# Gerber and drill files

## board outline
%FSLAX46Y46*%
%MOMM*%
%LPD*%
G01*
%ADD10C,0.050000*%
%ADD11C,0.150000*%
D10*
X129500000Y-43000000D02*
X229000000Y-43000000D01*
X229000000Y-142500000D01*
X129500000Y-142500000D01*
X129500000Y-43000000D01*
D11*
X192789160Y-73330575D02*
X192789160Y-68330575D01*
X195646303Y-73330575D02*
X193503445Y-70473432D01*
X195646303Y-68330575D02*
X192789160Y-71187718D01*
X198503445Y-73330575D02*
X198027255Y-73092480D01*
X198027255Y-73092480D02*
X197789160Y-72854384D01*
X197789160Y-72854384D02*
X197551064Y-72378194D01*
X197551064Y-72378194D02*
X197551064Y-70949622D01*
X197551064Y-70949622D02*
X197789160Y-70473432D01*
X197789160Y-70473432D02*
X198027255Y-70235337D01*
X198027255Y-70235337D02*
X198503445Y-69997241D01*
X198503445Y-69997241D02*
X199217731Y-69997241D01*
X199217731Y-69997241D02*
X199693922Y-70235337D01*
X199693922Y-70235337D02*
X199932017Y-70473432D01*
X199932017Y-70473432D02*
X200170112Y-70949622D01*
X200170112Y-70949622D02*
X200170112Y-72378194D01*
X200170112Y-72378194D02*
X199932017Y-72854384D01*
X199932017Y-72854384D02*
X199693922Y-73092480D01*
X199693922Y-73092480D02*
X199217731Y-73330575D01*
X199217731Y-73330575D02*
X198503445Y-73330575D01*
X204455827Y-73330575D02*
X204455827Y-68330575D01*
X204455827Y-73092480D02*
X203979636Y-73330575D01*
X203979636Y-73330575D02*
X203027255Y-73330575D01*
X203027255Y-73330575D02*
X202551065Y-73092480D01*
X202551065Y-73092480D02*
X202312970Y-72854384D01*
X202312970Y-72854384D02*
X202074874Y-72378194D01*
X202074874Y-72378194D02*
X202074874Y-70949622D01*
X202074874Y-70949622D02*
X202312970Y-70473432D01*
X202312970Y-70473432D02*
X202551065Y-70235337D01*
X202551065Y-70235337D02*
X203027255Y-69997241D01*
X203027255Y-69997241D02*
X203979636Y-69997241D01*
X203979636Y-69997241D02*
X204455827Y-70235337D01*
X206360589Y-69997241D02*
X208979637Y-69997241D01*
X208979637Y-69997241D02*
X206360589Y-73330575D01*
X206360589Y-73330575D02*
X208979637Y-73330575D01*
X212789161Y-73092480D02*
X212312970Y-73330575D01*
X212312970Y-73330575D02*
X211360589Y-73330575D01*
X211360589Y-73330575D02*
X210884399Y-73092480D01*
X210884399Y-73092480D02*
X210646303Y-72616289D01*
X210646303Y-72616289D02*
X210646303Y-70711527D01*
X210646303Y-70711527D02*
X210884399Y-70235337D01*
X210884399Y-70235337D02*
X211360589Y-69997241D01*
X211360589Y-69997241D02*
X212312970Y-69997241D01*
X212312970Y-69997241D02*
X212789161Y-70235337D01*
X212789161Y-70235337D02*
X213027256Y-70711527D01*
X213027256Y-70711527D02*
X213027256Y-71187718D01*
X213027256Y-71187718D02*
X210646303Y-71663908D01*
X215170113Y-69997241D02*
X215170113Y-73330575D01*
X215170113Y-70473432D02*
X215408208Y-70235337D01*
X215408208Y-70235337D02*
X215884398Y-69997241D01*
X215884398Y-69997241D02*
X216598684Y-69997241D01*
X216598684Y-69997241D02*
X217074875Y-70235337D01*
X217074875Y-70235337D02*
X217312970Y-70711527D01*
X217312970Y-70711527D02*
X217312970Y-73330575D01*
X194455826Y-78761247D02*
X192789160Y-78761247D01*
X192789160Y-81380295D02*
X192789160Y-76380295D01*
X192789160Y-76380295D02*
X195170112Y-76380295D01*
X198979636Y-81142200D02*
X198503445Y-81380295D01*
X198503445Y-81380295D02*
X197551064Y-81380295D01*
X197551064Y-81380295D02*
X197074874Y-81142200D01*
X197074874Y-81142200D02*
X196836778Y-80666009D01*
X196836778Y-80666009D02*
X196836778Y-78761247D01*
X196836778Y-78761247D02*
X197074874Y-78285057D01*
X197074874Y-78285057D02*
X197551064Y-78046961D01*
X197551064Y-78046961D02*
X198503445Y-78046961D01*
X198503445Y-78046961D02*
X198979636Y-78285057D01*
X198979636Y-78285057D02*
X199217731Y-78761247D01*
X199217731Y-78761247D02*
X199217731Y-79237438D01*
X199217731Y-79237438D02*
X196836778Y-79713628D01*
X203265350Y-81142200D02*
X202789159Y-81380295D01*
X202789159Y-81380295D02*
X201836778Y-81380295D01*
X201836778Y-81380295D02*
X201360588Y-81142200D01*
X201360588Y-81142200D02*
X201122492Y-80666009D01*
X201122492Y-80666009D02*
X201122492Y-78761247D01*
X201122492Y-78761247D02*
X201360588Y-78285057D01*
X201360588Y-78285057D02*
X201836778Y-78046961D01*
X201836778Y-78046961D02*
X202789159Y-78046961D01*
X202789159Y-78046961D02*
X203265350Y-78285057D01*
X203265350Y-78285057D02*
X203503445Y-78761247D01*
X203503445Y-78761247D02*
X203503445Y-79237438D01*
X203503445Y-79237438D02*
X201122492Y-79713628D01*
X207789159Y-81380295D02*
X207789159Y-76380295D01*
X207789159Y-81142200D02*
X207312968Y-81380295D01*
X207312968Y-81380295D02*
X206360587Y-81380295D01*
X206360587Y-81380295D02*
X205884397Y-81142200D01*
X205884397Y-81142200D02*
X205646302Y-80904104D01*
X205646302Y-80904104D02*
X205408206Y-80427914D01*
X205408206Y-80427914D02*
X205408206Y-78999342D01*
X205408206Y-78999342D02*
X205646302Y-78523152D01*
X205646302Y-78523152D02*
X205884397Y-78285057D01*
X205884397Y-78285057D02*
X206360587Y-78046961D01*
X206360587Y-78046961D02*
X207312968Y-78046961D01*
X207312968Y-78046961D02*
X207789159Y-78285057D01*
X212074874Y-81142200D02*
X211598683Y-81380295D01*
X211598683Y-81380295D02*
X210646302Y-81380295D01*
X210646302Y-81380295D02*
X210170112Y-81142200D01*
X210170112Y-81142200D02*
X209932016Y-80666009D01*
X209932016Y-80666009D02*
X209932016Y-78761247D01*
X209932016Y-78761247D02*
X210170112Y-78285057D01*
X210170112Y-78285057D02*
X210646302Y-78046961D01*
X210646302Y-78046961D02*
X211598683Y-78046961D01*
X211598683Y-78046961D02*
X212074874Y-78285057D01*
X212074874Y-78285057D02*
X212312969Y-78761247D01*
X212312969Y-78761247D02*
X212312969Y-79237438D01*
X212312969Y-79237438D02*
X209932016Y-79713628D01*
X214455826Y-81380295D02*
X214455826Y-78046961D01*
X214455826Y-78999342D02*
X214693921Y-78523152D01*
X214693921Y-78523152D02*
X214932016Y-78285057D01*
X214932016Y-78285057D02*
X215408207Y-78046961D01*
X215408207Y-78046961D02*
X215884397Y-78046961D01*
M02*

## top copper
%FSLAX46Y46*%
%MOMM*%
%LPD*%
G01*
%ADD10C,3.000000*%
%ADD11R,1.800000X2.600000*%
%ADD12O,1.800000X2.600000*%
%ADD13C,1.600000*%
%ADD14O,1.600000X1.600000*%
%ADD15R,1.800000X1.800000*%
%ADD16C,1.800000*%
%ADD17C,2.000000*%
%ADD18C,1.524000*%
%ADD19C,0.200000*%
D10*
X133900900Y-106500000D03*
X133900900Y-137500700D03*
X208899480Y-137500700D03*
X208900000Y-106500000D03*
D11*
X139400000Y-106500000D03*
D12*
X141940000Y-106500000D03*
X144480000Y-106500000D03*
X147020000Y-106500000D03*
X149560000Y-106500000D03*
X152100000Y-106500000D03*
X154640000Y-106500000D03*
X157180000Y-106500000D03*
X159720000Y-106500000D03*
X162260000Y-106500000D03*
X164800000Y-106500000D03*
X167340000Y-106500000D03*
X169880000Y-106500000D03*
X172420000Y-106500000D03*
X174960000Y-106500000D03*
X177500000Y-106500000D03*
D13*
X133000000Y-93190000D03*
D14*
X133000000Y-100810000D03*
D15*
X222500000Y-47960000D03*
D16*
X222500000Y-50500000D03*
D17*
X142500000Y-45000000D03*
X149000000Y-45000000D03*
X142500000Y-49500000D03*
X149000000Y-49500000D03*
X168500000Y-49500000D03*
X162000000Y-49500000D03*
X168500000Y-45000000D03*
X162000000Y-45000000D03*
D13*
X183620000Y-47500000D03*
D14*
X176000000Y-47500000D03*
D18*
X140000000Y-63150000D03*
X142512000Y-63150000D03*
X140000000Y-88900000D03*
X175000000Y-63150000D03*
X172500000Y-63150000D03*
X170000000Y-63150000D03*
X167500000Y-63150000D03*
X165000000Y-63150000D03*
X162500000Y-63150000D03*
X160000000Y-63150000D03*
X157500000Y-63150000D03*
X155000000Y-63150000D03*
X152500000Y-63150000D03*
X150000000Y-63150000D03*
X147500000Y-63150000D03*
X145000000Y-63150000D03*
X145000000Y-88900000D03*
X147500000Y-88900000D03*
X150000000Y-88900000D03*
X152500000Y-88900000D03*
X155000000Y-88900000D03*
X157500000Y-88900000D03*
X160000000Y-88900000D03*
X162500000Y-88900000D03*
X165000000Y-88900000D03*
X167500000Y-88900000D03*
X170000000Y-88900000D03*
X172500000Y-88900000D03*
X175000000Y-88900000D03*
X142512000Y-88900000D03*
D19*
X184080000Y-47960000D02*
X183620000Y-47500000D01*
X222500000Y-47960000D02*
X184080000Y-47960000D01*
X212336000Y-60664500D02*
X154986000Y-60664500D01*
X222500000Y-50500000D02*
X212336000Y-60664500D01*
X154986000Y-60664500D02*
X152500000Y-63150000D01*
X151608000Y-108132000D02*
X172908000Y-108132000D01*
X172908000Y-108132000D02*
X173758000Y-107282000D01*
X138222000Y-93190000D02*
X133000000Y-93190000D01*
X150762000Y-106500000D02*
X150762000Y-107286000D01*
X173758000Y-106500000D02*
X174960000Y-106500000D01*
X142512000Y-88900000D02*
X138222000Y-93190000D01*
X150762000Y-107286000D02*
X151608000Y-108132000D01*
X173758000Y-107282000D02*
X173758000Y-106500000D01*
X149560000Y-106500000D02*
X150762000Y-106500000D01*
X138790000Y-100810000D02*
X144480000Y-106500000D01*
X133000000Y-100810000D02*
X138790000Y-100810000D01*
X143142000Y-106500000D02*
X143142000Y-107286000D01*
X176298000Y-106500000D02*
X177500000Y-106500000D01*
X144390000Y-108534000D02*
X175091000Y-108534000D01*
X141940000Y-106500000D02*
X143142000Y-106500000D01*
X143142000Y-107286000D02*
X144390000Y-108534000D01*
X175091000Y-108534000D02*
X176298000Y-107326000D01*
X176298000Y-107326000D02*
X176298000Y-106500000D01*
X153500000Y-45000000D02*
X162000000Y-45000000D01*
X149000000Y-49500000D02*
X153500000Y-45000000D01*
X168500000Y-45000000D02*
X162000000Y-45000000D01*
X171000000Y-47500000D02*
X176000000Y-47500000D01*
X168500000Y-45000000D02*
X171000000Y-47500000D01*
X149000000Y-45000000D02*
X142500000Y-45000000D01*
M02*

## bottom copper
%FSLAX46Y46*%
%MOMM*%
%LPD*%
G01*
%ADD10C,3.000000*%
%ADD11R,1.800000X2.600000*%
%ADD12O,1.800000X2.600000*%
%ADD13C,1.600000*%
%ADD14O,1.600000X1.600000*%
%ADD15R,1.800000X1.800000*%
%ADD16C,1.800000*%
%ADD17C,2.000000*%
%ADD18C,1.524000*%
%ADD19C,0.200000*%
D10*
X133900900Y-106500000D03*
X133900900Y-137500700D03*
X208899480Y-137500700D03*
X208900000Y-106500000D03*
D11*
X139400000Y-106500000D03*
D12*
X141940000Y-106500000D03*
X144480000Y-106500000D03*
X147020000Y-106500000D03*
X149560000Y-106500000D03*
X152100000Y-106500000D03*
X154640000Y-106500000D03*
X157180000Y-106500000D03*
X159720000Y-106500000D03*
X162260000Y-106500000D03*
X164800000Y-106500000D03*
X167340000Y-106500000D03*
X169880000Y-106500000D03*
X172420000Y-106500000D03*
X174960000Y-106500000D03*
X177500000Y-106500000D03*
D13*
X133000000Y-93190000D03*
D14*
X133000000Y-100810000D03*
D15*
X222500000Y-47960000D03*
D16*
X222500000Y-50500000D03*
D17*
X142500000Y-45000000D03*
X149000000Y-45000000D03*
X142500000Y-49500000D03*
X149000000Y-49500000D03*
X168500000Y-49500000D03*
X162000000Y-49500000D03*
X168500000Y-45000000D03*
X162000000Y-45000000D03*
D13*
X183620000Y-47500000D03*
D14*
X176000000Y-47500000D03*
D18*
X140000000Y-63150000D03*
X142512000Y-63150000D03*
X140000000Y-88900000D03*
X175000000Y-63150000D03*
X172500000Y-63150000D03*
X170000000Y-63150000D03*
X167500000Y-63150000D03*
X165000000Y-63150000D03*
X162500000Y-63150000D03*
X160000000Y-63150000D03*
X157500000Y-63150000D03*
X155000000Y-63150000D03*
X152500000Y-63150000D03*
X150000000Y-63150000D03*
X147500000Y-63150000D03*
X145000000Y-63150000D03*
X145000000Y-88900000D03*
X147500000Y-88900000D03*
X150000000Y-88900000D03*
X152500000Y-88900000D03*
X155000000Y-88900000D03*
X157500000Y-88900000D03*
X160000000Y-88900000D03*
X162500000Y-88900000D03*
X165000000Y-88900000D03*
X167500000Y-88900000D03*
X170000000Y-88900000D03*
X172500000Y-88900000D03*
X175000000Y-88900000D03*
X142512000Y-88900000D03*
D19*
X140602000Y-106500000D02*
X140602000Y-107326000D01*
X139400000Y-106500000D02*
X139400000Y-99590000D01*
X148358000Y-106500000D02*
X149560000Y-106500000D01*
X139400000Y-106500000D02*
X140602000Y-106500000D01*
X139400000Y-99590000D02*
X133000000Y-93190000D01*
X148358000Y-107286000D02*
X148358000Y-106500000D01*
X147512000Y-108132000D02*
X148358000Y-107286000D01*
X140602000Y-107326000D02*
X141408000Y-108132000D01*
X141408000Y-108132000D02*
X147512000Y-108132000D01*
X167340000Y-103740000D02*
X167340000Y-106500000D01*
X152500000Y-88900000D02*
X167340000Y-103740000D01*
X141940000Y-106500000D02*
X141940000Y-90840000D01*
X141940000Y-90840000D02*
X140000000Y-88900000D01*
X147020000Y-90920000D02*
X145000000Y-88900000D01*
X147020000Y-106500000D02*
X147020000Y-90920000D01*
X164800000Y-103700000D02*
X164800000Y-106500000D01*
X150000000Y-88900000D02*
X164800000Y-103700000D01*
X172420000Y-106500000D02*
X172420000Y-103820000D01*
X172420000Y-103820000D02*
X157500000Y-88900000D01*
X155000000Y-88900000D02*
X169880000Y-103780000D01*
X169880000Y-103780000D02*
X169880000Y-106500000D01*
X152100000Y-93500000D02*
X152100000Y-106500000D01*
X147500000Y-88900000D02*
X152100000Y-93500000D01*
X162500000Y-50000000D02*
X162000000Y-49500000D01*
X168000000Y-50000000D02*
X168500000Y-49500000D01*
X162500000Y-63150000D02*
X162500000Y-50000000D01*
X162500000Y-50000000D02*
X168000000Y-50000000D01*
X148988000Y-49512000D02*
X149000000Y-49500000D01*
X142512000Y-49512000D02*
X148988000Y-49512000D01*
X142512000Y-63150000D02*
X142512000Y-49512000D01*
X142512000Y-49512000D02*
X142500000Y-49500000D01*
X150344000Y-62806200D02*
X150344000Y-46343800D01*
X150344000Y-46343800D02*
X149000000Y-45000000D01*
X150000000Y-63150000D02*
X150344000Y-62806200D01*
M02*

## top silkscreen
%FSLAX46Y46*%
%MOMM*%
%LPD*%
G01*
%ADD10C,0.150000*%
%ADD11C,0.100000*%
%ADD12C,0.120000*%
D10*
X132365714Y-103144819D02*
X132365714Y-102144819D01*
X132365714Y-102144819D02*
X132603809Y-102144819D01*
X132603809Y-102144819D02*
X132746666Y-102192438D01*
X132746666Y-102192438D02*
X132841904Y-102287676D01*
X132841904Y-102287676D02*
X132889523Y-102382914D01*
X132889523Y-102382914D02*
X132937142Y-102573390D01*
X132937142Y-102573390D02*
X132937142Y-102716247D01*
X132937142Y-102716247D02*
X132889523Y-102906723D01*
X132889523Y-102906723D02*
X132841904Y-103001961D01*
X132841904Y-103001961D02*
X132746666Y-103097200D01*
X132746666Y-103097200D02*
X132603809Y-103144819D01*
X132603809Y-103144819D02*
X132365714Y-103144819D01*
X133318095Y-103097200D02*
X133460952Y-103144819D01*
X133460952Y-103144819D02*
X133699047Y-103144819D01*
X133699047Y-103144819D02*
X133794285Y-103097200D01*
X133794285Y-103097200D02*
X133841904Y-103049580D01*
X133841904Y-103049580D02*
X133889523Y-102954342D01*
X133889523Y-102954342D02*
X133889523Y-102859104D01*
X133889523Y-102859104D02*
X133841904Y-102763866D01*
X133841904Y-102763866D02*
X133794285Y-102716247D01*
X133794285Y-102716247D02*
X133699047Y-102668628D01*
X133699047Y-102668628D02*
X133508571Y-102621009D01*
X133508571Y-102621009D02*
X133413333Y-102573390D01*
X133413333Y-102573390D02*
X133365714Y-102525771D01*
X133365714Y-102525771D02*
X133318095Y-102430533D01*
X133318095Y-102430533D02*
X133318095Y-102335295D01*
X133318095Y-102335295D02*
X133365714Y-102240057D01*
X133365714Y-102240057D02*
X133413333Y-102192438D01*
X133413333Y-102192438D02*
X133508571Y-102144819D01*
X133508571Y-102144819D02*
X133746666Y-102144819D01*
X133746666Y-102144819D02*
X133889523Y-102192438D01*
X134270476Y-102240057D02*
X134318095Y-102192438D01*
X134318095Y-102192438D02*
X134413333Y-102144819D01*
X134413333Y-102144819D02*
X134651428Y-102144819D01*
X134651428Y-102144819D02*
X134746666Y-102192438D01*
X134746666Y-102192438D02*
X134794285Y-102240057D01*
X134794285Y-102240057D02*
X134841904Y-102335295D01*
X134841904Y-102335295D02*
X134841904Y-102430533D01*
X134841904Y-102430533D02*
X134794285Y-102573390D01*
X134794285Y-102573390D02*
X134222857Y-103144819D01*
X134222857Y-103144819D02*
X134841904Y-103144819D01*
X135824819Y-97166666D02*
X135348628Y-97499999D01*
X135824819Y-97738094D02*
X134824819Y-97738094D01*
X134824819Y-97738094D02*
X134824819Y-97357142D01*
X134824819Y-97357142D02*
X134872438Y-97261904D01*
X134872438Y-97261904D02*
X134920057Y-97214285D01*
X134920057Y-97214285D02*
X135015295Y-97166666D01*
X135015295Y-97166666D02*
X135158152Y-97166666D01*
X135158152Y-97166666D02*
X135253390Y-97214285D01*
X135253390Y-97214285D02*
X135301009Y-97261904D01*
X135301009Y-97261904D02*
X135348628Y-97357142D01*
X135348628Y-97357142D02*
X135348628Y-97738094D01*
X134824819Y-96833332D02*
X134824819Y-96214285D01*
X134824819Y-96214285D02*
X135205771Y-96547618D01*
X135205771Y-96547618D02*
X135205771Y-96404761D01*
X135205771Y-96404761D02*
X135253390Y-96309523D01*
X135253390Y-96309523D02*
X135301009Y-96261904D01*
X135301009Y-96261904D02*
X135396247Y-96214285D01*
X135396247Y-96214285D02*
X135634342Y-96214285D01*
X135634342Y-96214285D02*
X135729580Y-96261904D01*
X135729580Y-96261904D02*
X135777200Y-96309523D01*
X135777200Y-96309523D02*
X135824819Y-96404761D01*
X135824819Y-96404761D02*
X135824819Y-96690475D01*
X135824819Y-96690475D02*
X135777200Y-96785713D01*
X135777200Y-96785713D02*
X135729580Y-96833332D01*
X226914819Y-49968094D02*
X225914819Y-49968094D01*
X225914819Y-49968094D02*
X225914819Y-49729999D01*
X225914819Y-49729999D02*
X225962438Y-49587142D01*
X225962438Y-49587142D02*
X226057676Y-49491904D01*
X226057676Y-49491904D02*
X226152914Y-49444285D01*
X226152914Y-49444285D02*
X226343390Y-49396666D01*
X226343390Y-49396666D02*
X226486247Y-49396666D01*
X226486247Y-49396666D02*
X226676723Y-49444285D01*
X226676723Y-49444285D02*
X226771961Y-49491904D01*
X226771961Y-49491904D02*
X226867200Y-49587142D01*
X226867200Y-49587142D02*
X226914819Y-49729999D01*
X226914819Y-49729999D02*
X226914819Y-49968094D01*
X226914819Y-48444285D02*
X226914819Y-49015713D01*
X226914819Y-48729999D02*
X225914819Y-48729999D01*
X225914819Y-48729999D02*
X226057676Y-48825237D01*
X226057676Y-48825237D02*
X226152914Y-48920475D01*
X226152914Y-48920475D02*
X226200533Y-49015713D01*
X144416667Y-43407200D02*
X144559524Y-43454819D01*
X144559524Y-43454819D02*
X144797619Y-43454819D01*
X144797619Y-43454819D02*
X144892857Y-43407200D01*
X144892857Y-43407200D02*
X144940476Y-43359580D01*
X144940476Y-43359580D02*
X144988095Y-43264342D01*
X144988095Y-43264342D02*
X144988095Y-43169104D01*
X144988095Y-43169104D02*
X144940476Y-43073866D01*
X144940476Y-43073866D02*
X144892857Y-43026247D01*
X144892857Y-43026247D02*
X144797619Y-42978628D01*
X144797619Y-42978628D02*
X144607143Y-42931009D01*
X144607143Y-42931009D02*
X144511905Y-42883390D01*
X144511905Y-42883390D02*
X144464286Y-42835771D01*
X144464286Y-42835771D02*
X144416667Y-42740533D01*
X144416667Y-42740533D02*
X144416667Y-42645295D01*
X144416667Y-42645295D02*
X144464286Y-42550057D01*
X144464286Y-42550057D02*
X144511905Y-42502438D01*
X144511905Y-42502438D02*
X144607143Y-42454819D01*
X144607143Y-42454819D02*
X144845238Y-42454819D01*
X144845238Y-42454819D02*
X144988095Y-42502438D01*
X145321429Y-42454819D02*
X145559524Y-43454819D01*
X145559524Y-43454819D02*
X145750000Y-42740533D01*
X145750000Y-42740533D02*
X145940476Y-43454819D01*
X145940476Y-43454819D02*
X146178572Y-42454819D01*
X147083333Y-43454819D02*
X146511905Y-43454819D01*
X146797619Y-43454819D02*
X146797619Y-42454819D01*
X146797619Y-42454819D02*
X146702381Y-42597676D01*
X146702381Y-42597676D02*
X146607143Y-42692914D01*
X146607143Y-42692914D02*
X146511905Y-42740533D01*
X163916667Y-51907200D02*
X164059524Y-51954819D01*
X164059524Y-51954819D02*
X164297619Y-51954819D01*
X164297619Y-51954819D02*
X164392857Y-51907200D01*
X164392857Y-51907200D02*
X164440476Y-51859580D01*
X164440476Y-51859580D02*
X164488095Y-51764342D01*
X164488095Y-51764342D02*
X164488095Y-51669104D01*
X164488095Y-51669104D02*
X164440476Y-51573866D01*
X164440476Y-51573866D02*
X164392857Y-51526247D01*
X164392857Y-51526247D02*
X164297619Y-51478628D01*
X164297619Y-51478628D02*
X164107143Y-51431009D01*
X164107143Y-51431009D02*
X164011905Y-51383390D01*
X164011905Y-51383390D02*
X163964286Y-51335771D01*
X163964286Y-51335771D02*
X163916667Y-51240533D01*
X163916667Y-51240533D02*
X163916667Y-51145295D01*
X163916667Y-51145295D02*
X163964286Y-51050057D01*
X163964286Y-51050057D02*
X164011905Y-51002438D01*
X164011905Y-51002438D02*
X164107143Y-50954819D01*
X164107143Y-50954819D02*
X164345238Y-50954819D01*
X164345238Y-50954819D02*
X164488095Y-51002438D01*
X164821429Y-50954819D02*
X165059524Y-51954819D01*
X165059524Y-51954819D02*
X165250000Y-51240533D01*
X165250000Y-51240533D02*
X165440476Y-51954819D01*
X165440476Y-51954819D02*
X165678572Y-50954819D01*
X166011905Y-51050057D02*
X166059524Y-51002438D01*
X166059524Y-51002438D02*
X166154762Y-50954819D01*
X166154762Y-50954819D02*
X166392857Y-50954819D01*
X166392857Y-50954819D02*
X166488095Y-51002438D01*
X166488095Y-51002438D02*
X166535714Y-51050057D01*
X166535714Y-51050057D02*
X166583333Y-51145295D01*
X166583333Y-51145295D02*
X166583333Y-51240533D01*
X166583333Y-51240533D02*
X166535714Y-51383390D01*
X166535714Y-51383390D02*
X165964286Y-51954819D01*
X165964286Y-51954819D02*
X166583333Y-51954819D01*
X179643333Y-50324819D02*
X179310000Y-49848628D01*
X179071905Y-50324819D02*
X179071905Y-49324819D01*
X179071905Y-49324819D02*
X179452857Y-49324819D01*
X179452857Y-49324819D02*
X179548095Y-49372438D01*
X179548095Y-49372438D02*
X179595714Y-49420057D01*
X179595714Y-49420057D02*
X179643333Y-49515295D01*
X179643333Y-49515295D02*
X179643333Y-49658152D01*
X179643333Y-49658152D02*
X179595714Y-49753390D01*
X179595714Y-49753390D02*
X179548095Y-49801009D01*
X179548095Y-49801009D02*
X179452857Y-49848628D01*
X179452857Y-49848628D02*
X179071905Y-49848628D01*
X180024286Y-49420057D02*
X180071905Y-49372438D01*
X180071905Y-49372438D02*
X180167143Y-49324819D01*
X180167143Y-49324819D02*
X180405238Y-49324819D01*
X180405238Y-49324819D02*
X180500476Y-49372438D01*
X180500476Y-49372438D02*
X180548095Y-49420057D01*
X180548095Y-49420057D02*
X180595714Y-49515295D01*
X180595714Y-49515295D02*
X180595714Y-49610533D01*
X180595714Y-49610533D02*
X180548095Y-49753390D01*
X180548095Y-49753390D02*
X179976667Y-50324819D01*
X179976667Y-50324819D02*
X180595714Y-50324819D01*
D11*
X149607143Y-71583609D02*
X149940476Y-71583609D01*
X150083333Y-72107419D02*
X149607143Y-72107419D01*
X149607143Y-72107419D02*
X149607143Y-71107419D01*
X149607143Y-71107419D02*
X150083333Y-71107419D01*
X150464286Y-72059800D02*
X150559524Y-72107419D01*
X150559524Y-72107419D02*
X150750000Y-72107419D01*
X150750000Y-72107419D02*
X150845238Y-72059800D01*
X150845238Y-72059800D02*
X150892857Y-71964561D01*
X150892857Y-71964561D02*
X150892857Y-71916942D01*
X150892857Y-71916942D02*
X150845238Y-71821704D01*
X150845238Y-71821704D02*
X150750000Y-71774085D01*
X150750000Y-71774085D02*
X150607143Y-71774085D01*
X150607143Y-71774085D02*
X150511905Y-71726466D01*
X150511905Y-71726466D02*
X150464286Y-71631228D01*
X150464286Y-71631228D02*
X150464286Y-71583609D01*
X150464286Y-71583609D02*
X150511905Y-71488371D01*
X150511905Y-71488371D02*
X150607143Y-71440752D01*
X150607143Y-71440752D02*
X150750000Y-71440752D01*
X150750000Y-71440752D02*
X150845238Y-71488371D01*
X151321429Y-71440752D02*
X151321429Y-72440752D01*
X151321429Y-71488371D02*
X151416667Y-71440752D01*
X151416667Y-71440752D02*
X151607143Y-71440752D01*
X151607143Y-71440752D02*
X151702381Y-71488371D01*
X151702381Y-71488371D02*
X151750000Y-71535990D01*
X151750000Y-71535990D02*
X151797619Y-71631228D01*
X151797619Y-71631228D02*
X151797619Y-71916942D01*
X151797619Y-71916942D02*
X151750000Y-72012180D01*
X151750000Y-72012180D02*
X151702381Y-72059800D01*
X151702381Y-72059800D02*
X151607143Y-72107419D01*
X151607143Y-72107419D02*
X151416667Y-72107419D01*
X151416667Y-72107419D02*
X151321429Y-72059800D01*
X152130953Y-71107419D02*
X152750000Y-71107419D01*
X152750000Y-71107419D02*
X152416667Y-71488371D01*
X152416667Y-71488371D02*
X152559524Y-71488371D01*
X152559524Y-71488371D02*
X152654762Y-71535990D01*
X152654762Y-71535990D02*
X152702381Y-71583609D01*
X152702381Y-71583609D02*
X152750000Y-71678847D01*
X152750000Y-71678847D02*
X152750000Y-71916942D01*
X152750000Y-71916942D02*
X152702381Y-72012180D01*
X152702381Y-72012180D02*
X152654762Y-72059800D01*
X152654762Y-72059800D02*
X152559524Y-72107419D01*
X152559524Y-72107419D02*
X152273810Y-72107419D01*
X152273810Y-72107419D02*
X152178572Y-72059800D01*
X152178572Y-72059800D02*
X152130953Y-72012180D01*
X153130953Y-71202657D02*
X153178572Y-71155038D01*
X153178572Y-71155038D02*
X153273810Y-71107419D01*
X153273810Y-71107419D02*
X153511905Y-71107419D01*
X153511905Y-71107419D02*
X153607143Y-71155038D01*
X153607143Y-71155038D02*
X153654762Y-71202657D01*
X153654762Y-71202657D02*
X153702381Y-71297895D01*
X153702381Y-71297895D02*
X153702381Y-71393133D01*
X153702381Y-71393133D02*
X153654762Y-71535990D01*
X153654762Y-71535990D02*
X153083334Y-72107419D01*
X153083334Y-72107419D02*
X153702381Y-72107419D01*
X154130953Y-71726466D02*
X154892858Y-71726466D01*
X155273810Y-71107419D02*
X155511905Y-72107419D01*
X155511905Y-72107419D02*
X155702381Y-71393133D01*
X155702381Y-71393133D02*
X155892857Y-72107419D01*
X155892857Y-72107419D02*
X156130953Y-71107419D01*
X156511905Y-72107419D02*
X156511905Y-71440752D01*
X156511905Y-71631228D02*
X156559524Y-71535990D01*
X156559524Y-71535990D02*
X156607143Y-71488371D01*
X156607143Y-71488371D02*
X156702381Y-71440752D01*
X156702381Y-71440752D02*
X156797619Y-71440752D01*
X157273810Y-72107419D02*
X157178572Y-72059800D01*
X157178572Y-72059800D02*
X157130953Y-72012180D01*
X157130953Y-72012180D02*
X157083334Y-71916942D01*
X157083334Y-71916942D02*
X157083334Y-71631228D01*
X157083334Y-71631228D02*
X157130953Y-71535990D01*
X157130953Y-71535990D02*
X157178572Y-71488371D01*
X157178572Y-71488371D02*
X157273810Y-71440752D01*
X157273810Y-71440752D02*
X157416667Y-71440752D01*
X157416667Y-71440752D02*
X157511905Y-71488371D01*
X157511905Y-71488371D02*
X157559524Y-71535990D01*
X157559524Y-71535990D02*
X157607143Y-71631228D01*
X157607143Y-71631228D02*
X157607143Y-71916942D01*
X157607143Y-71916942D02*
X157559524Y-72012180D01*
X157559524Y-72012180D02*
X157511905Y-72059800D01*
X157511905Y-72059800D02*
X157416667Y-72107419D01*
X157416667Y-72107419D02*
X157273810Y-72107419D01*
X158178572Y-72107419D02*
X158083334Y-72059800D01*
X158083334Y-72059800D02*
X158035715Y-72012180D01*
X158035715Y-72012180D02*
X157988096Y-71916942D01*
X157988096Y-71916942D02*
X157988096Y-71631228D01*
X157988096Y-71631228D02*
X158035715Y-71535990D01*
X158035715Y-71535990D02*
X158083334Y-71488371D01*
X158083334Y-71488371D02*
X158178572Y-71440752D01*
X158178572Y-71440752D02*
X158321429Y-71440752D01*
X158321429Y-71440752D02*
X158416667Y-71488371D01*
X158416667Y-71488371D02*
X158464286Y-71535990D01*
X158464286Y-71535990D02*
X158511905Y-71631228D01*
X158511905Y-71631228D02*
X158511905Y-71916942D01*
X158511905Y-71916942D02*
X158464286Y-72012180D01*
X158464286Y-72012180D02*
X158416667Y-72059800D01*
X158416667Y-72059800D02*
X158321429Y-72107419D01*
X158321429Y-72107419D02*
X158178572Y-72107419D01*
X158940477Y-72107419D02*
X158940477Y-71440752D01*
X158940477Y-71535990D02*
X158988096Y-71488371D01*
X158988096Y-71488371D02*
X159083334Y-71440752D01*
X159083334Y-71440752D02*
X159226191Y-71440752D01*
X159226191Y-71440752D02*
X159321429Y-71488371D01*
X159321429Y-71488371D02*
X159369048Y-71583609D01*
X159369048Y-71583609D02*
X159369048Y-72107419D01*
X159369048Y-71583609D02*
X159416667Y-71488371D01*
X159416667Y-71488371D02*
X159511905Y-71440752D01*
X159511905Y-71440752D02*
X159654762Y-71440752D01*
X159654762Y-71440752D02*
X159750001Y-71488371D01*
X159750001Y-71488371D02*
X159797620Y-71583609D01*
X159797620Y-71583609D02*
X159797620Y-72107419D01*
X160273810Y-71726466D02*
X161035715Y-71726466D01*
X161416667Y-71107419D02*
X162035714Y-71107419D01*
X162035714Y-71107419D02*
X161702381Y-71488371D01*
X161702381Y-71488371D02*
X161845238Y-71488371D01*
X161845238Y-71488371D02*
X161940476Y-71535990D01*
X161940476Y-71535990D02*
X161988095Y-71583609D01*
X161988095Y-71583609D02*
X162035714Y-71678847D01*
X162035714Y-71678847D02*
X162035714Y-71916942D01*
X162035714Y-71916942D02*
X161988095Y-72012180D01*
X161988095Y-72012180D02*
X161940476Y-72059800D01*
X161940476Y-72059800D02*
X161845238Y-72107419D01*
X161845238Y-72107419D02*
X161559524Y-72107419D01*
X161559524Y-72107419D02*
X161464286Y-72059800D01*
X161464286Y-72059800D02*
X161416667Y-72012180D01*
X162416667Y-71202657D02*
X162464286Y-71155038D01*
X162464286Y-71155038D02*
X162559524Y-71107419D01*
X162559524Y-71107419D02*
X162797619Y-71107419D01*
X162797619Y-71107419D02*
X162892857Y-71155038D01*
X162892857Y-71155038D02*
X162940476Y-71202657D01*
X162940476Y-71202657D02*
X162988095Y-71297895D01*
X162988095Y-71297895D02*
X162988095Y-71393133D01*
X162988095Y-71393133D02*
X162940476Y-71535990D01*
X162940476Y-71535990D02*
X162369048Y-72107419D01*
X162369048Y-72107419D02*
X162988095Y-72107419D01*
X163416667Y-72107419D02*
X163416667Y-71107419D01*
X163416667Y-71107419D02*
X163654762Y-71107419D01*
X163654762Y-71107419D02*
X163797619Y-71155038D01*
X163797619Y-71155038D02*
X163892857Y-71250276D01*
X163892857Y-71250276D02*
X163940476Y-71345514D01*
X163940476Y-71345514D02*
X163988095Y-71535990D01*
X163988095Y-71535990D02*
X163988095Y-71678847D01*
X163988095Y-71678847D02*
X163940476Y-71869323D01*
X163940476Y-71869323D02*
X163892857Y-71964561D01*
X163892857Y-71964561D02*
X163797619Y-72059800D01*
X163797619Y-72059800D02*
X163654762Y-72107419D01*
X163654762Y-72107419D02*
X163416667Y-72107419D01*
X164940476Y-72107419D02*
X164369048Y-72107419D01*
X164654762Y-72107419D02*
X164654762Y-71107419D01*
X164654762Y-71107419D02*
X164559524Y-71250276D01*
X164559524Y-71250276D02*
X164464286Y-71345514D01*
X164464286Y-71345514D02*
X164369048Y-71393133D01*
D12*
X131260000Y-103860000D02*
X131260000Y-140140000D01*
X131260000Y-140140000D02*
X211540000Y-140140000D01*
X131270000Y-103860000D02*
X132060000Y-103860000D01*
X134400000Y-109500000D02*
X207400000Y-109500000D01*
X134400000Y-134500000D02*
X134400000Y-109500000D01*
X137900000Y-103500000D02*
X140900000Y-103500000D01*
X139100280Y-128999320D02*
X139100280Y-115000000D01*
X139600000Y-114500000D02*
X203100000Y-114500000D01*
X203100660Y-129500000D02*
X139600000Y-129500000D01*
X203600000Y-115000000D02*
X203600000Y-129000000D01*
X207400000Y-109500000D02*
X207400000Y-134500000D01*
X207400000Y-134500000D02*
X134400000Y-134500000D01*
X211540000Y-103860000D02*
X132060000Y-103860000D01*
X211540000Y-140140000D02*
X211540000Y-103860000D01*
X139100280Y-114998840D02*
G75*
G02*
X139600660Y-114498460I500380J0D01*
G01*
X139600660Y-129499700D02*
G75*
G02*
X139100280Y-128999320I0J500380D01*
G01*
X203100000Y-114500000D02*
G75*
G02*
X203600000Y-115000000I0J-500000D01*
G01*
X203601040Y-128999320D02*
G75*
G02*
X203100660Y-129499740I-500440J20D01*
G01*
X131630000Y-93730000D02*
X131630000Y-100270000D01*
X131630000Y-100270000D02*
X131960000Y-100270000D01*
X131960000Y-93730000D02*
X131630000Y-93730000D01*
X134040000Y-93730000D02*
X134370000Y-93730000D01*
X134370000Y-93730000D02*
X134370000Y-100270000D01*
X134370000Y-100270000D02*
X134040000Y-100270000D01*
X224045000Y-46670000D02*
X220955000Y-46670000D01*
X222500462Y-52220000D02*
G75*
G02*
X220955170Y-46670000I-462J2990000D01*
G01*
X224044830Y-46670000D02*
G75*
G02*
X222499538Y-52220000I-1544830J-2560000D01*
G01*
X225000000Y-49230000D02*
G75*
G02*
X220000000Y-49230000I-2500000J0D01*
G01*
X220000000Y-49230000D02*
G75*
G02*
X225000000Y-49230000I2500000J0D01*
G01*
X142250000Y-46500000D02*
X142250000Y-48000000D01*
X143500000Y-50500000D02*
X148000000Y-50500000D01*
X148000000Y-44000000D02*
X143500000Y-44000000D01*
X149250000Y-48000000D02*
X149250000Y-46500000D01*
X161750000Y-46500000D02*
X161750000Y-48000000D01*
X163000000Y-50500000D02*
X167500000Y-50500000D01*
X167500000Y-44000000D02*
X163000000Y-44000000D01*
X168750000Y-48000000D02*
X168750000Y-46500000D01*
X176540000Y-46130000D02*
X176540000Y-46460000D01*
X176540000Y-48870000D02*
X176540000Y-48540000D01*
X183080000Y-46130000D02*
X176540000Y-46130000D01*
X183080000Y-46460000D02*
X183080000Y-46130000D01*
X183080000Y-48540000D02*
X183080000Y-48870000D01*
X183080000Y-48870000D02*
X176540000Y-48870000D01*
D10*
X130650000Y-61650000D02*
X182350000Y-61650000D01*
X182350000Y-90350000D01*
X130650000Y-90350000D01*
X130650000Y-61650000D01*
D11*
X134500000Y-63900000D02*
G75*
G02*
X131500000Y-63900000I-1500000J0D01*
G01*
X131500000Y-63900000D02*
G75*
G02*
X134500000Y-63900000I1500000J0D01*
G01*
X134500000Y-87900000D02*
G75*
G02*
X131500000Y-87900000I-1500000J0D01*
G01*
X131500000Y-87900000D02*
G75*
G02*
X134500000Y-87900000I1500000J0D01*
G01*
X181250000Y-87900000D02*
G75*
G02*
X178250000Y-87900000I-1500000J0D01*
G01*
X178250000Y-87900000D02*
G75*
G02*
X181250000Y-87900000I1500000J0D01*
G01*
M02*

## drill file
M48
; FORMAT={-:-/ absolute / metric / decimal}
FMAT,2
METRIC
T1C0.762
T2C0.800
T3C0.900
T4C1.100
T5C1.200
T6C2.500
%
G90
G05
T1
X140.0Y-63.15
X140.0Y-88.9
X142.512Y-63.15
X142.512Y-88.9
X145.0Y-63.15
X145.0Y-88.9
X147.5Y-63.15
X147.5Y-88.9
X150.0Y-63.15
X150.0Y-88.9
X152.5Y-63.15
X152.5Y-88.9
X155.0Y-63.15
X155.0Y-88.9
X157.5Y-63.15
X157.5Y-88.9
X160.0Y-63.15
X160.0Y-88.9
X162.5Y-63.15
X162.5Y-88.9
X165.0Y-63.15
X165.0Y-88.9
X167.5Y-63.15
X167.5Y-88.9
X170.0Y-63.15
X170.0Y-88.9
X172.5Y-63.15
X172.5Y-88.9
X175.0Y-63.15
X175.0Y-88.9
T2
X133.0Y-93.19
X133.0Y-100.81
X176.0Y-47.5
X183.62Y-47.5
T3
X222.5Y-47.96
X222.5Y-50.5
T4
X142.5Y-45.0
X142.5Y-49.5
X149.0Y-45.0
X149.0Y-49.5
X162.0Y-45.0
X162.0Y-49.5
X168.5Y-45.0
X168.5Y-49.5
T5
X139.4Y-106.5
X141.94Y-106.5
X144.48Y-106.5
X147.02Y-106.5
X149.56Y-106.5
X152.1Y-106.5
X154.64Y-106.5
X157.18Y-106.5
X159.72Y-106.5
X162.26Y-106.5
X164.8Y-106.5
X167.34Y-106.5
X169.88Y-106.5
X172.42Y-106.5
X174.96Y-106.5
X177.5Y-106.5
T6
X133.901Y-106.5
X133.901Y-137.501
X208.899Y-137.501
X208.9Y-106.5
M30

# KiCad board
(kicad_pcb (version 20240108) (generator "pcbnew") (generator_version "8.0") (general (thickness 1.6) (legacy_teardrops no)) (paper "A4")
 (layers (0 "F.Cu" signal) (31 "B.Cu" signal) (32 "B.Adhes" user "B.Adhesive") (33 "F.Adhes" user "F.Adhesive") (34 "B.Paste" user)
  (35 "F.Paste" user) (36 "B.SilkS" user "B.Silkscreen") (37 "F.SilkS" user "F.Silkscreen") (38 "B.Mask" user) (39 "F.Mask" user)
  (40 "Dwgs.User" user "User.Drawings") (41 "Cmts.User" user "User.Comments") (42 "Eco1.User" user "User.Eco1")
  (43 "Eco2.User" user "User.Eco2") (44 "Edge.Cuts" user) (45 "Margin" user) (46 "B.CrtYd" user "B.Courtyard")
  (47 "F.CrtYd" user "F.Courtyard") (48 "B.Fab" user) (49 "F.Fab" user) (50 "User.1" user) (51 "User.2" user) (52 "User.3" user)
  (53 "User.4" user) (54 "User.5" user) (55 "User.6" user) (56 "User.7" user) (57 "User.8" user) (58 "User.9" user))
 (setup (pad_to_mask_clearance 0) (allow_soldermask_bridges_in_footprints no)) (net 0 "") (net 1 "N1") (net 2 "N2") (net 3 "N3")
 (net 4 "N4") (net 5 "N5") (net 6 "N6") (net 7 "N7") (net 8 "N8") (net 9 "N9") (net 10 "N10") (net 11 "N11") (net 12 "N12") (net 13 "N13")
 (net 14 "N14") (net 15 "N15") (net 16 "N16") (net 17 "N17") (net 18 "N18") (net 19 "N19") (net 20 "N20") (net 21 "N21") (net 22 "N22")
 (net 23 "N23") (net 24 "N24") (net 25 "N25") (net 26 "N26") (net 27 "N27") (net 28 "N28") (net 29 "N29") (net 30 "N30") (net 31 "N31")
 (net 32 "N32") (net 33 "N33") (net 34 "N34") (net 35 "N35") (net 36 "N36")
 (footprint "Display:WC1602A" (layer "F.Cu") (at 139.4 106.5)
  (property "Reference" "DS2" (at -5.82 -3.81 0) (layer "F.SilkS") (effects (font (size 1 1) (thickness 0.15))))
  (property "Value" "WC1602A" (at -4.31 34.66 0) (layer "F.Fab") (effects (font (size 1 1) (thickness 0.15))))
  (fp_line (start -8.14 -2.64) (end -8.14 33.64) (stroke (width 0.12) (type solid)) (layer "F.SilkS"))
  (fp_line (start -8.14 33.64) (end 72.14 33.64) (stroke (width 0.12) (type solid)) (layer "F.SilkS"))
  (fp_line (start -8.13 -2.64) (end -7.34 -2.64) (stroke (width 0.12) (type solid)) (layer "F.SilkS"))
  (fp_line (start -5 3) (end 68 3) (stroke (width 0.12) (type solid)) (layer "F.SilkS"))
  (fp_line (start -5 28) (end -5 3) (stroke (width 0.12) (type solid)) (layer "F.SilkS"))
  (fp_line (start -1.5 -3) (end 1.5 -3) (stroke (width 0.12) (type solid)) (layer "F.SilkS"))
  (fp_line (start -0.29972 22.49932) (end -0.29972 8.5) (stroke (width 0.12) (type solid)) (layer "F.SilkS"))
  (fp_line (start 0.2 8) (end 63.7 8) (stroke (width 0.12) (type solid)) (layer "F.SilkS"))
  (fp_line (start 63.70066 23) (end 0.2 23) (stroke (width 0.12) (type solid)) (layer "F.SilkS"))
  (fp_line (start 64.2 8.5) (end 64.2 22.5) (stroke (width 0.12) (type solid)) (layer "F.SilkS"))
  (fp_line (start 68 3) (end 68 28) (stroke (width 0.12) (type solid)) (layer "F.SilkS"))
  (fp_line (start 68 28) (end -5 28) (stroke (width 0.12) (type solid)) (layer "F.SilkS"))
  (fp_line (start 72.14 -2.64) (end -7.34 -2.64) (stroke (width 0.12) (type solid)) (layer "F.SilkS"))
  (fp_line (start 72.14 33.64) (end 72.14 -2.64) (stroke (width 0.12) (type solid)) (layer "F.SilkS"))
  (fp_arc (start -0.29972 8.49884) (mid -0.153162 8.145018) (end 0.20066 7.99846) (stroke (width 0.12) (type solid)) (layer "F.SilkS"))
  (fp_arc (start 0.20066 22.9997) (mid -0.153162 22.853142) (end -0.29972 22.49932) (stroke (width 0.12) (type solid)) (layer "F.SilkS"))
  (fp_arc (start 63.7 8) (mid 64.053553 8.146447) (end 64.2 8.5) (stroke (width 0.12) (type solid)) (layer "F.SilkS"))
  (fp_arc (start 64.20104 22.49932) (mid 64.054473 22.853115) (end 63.70066 22.9997) (stroke (width 0.12) (type solid)) (layer "F.SilkS"))
  (pad "" thru_hole circle (at -5.4991 0) (size 3 3) (drill 2.5) (layers "*.Cu" "*.Mask") (remove_unused_layers no))
  (pad "" thru_hole circle (at -5.4991 31.0007) (size 3 3) (drill 2.5) (layers "*.Cu" "*.Mask") (remove_unused_layers no))
  (pad "" thru_hole circle (at 69.49948 31.0007) (size 3 3) (drill 2.5) (layers "*.Cu" "*.Mask") (remove_unused_layers no))
  (pad "" thru_hole circle (at 69.5 0) (size 3 3) (drill 2.5) (layers "*.Cu" "*.Mask") (remove_unused_layers no))
  (pad "1" thru_hole rect (at 0 0) (size 1.8 2.6) (drill 1.2) (layers "*.Cu" "*.Mask") (remove_unused_layers no) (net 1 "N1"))
  (pad "2" thru_hole oval (at 2.54 0) (size 1.8 2.6) (drill 1.2) (layers "*.Cu" "*.Mask") (remove_unused_layers no) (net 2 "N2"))
  (pad "3" thru_hole oval (at 5.08 0) (size 1.8 2.6) (drill 1.2) (layers "*.Cu" "*.Mask") (remove_unused_layers no) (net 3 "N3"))
  (pad "4" thru_hole oval (at 7.62 0) (size 1.8 2.6) (drill 1.2) (layers "*.Cu" "*.Mask") (remove_unused_layers no) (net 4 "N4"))
  (pad "5" thru_hole oval (at 10.16 0) (size 1.8 2.6) (drill 1.2) (layers "*.Cu" "*.Mask") (remove_unused_layers no) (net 1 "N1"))
  (pad "6" thru_hole oval (at 12.7 0) (size 1.8 2.6) (drill 1.2) (layers "*.Cu" "*.Mask") (remove_unused_layers no) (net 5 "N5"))
  (pad "7" thru_hole oval (at 15.24 0) (size 1.8 2.6) (drill 1.2) (layers "*.Cu" "*.Mask") (remove_unused_layers no) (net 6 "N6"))
  (pad "8" thru_hole oval (at 17.78 0) (size 1.8 2.6) (drill 1.2) (layers "*.Cu" "*.Mask") (remove_unused_layers no) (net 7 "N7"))
  (pad "9" thru_hole oval (at 20.32 0) (size 1.8 2.6) (drill 1.2) (layers "*.Cu" "*.Mask") (remove_unused_layers no) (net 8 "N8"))
  (pad "10" thru_hole oval (at 22.86 0) (size 1.8 2.6) (drill 1.2) (layers "*.Cu" "*.Mask") (remove_unused_layers no) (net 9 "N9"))
  (pad "11" thru_hole oval (at 25.4 0) (size 1.8 2.6) (drill 1.2) (layers "*.Cu" "*.Mask") (remove_unused_layers no) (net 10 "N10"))
  (pad "12" thru_hole oval (at 27.94 0) (size 1.8 2.6) (drill 1.2) (layers "*.Cu" "*.Mask") (remove_unused_layers no) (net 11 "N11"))
  (pad "13" thru_hole oval (at 30.48 0) (size 1.8 2.6) (drill 1.2) (layers "*.Cu" "*.Mask") (remove_unused_layers no) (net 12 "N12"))
  (pad "14" thru_hole oval (at 33.02 0) (size 1.8 2.6) (drill 1.2) (layers "*.Cu" "*.Mask") (remove_unused_layers no) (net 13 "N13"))
  (pad "15" thru_hole oval (at 35.56 0) (size 1.8 2.6) (drill 1.2) (layers "*.Cu" "*.Mask") (remove_unused_layers no) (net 1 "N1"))
  (pad "16" thru_hole oval (at 38.1 0) (size 1.8 2.6) (drill 1.2) (layers "*.Cu" "*.Mask") (remove_unused_layers no) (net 2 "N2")))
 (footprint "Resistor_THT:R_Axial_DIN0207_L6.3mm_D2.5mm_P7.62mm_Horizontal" (layer "F.Cu") (at 133 93.19 -90)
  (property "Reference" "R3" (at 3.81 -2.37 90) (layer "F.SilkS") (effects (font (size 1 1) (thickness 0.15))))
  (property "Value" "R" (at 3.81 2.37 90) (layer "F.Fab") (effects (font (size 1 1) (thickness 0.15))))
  (fp_line (start 0.54 1.37) (end 7.08 1.37) (stroke (width 0.12) (type solid)) (layer "F.SilkS"))
  (fp_line (start 7.08 1.37) (end 7.08 1.04) (stroke (width 0.12) (type solid)) (layer "F.SilkS"))
  (fp_line (start 0.54 1.04) (end 0.54 1.37) (stroke (width 0.12) (type solid)) (layer "F.SilkS"))
  (fp_line (start 0.54 -1.04) (end 0.54 -1.37) (stroke (width 0.12) (type solid)) (layer "F.SilkS"))
  (fp_line (start 0.54 -1.37) (end 7.08 -1.37) (stroke (width 0.12) (type solid)) (layer "F.SilkS"))
  (fp_line (start 7.08 -1.37) (end 7.08 -1.04) (stroke (width 0.12) (type solid)) (layer "F.SilkS"))
  (pad "1" thru_hole circle (at 0 0 270) (size 1.6 1.6) (drill 0.8) (layers "*.Cu" "*.Mask") (remove_unused_layers no) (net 1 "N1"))
  (pad "2" thru_hole oval (at 7.62 0 270) (size 1.6 1.6) (drill 0.8) (layers "*.Cu" "*.Mask") (remove_unused_layers no) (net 3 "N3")))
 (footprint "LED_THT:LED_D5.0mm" (layer "F.Cu") (at 222.5 47.96 -90)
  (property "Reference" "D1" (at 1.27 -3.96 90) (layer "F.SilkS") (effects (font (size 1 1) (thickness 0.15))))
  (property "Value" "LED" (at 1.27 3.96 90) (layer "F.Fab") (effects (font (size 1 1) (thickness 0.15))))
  (fp_line (start -1.29 -1.545) (end -1.29 1.545) (stroke (width 0.12) (type solid)) (layer "F.SilkS"))
  (fp_arc (start 4.26 -0.000462) (mid 2.072002 2.880433) (end -1.29 1.54483) (stroke (width 0.12) (type solid)) (layer "F.SilkS"))
  (fp_arc (start -1.29 -1.54483) (mid 2.072002 -2.880433) (end 4.26 0.000462) (stroke (width 0.12) (type solid)) (layer "F.SilkS"))
  (fp_circle (center 1.27 0) (end 3.77 0) (stroke (width 0.12) (type solid)) (fill none) (layer "F.SilkS"))
  (pad "1" thru_hole rect (at 0 0 270) (size 1.8 1.8) (drill 0.9) (layers "*.Cu" "*.Mask") (remove_unused_layers no) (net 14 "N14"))
  (pad "2" thru_hole circle (at 2.54 0 270) (size 1.8 1.8) (drill 0.9) (layers "*.Cu" "*.Mask") (remove_unused_layers no) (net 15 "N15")))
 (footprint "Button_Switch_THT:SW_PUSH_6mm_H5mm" (layer "F.Cu") (at 142.5 45)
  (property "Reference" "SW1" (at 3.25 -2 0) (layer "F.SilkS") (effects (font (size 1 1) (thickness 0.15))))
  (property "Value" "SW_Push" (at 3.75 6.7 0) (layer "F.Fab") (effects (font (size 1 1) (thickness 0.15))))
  (fp_line (start -0.25 1.5) (end -0.25 3) (stroke (width 0.12) (type solid)) (layer "F.SilkS"))
  (fp_line (start 1 5.5) (end 5.5 5.5) (stroke (width 0.12) (type solid)) (layer "F.SilkS"))
  (fp_line (start 5.5 -1) (end 1 -1) (stroke (width 0.12) (type solid)) (layer "F.SilkS"))
  (fp_line (start 6.75 3) (end 6.75 1.5) (stroke (width 0.12) (type solid)) (layer "F.SilkS"))
  (pad "1" thru_hole circle (at 0 0 90) (size 2 2) (drill 1.1) (layers "*.Cu" "*.Mask") (remove_unused_layers no) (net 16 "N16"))
  (pad "1" thru_hole circle (at 6.5 0 90) (size 2 2) (drill 1.1) (layers "*.Cu" "*.Mask") (remove_unused_layers no) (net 16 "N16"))
  (pad "2" thru_hole circle (at 0 4.5 90) (size 2 2) (drill 1.1) (layers "*.Cu" "*.Mask") (remove_unused_layers no) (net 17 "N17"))
  (pad "2" thru_hole circle (at 6.5 4.5 90) (size 2 2) (drill 1.1) (layers "*.Cu" "*.Mask") (remove_unused_layers no) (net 17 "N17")))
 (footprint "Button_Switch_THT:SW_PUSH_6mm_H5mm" (layer "F.Cu") (at 168.5 49.5 180)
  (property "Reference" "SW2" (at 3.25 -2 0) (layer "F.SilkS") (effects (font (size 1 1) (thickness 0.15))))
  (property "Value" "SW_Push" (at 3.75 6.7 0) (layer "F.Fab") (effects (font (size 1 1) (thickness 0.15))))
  (fp_line (start 6.75 3) (end 6.75 1.5) (stroke (width 0.12) (type solid)) (layer "F.SilkS"))
  (fp_line (start 5.5 -1) (end 1 -1) (stroke (width 0.12) (type solid)) (layer "F.SilkS"))
  (fp_line (start 1 5.5) (end 5.5 5.5) (stroke (width 0.12) (type solid)) (layer "F.SilkS"))
  (fp_line (start -0.25 1.5) (end -0.25 3) (stroke (width 0.12) (type solid)) (layer "F.SilkS"))
  (pad "1" thru_hole circle (at 0 0 270) (size 2 2) (drill 1.1) (layers "*.Cu" "*.Mask") (remove_unused_layers no) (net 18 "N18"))
  (pad "1" thru_hole circle (at 6.5 0 270) (size 2 2) (drill 1.1) (layers "*.Cu" "*.Mask") (remove_unused_layers no) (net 18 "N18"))
  (pad "2" thru_hole circle (at 0 4.5 270) (size 2 2) (drill 1.1) (layers "*.Cu" "*.Mask") (remove_unused_layers no) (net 17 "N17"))
  (pad "2" thru_hole circle (at 6.5 4.5 270) (size 2 2) (drill 1.1) (layers "*.Cu" "*.Mask") (remove_unused_layers no) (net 17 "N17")))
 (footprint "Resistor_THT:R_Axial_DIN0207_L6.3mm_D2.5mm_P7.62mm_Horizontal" (layer "F.Cu") (at 183.62 47.5 180)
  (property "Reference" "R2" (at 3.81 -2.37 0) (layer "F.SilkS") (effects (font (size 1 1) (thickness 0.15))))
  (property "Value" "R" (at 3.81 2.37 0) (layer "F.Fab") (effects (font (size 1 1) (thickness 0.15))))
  (fp_line (start 7.08 1.37) (end 7.08 1.04) (stroke (width 0.12) (type solid)) (layer "F.SilkS"))
  (fp_line (start 7.08 -1.37) (end 7.08 -1.04) (stroke (width 0.12) (type solid)) (layer "F.SilkS"))
  (fp_line (start 0.54 1.37) (end 7.08 1.37) (stroke (width 0.12) (type solid)) (layer "F.SilkS"))
  (fp_line (start 0.54 1.04) (end 0.54 1.37) (stroke (width 0.12) (type solid)) (layer "F.SilkS"))
  (fp_line (start 0.54 -1.04) (end 0.54 -1.37) (stroke (width 0.12) (type solid)) (layer "F.SilkS"))
  (fp_line (start 0.54 -1.37) (end 7.08 -1.37) (stroke (width 0.12) (type solid)) (layer "F.SilkS"))
  (pad "1" thru_hole circle (at 0 0 180) (size 1.6 1.6) (drill 0.8) (layers "*.Cu" "*.Mask") (remove_unused_layers no) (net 14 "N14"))
  (pad "2" thru_hole oval (at 7.62 0 180) (size 1.6 1.6) (drill 0.8) (layers "*.Cu" "*.Mask") (remove_unused_layers no) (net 17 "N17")))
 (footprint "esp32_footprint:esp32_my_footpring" (layer "F.Cu") (at 157.25 72.15)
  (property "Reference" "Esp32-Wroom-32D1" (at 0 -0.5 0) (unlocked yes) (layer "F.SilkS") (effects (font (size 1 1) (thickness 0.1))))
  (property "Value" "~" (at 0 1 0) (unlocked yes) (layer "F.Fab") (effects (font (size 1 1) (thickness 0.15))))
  (fp_rect (start -26.6 -10.5) (end 25.1 18.2) (stroke (width 0.15) (type default)) (fill none) (layer "F.SilkS"))
  (fp_circle (center -24.25 -8.25) (end -22.75 -8.25) (stroke (width 0.1) (type default)) (fill none) (layer "F.SilkS"))
  (fp_circle (center -24.25 15.75) (end -22.75 15.75) (stroke (width 0.1) (type default)) (fill none) (layer "F.SilkS"))
  (fp_circle (center 22.5 15.75) (end 24 15.75) (stroke (width 0.1) (type default)) (fill none) (layer "F.SilkS"))
  (pad "0" thru_hole circle (at -17.25 -9) (size 1.524 1.524) (drill 0.762) (layers "*.Cu" "*.Mask") (remove_unused_layers no)
   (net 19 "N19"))
  (pad "1" thru_hole circle (at -14.738 -9) (size 1.524 1.524) (drill 0.762) (layers "*.Cu" "*.Mask") (remove_unused_layers no)
   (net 17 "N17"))
  (pad "2" thru_hole circle (at -17.25 16.75) (size 1.524 1.524) (drill 0.762) (layers "*.Cu" "*.Mask") (remove_unused_layers no)
   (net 2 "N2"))
  (pad "3" thru_hole circle (at 17.75 -9) (size 1.524 1.524) (drill 0.762) (layers "*.Cu" "*.Mask") (remove_unused_layers no) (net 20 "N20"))
  (pad "4" thru_hole circle (at 15.25 -9) (size 1.524 1.524) (drill 0.762) (layers "*.Cu" "*.Mask") (remove_unused_layers no) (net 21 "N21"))
  (pad "5" thru_hole circle (at 12.75 -9) (size 1.524 1.524) (drill 0.762) (layers "*.Cu" "*.Mask") (remove_unused_layers no) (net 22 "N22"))
  (pad "6" thru_hole circle (at 10.25 -9) (size 1.524 1.524) (drill 0.762) (layers "*.Cu" "*.Mask") (remove_unused_layers no) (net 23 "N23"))
  (pad "7" thru_hole circle (at 7.75 -9) (size 1.524 1.524) (drill 0.762) (layers "*.Cu" "*.Mask") (remove_unused_layers no) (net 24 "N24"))
  (pad "8" thru_hole circle (at 5.25 -9) (size 1.524 1.524) (drill 0.762) (layers "*.Cu" "*.Mask") (remove_unused_layers no) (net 18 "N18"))
  (pad "9" thru_hole circle (at 2.75 -9) (size 1.524 1.524) (drill 0.762) (layers "*.Cu" "*.Mask") (remove_unused_layers no) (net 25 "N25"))
  (pad "10" thru_hole circle (at 0.25 -9) (size 1.524 1.524) (drill 0.762) (layers "*.Cu" "*.Mask") (remove_unused_layers no) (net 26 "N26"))
  (pad "11" thru_hole circle (at -2.25 -9) (size 1.524 1.524) (drill 0.762) (layers "*.Cu" "*.Mask") (remove_unused_layers no)
   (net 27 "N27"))
  (pad "12" thru_hole circle (at -4.75 -9) (size 1.524 1.524) (drill 0.762) (layers "*.Cu" "*.Mask") (remove_unused_layers no)
   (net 15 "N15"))
  (pad "13" thru_hole circle (at -7.25 -9) (size 1.524 1.524) (drill 0.762) (layers "*.Cu" "*.Mask") (remove_unused_layers no)
   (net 16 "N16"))
  (pad "14" thru_hole circle (at -9.75 -9) (size 1.524 1.524) (drill 0.762) (layers "*.Cu" "*.Mask") (remove_unused_layers no)
   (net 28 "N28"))
  (pad "16" thru_hole circle (at -12.25 -9) (size 1.524 1.524) (drill 0.762) (layers "*.Cu" "*.Mask") (remove_unused_layers no)
   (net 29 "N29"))
  (pad "23" thru_hole circle (at -12.25 16.75) (size 1.524 1.524) (drill 0.762) (layers "*.Cu" "*.Mask") (remove_unused_layers no)
   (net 4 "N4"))
  (pad "24" thru_hole circle (at -9.75 16.75) (size 1.524 1.524) (drill 0.762) (layers "*.Cu" "*.Mask") (remove_unused_layers no)
   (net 5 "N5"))
  (pad "26" thru_hole circle (at -7.25 16.75) (size 1.524 1.524) (drill 0.762) (layers "*.Cu" "*.Mask") (remove_unused_layers no)
   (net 10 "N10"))
  (pad "27" thru_hole circle (at -4.75 16.75) (size 1.524 1.524) (drill 0.762) (layers "*.Cu" "*.Mask") (remove_unused_layers no)
   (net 11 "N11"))
  (pad "28" thru_hole circle (at -2.25 16.75) (size 1.524 1.524) (drill 0.762) (layers "*.Cu" "*.Mask") (remove_unused_layers no)
   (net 12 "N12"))
  (pad "29" thru_hole circle (at 0.25 16.75) (size 1.524 1.524) (drill 0.762) (layers "*.Cu" "*.Mask") (remove_unused_layers no)
   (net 13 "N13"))
  (pad "30" thru_hole circle (at 2.75 16.75) (size 1.524 1.524) (drill 0.762) (layers "*.Cu" "*.Mask") (remove_unused_layers no)
   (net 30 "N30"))
  (pad "31" thru_hole circle (at 5.25 16.75) (size 1.524 1.524) (drill 0.762) (layers "*.Cu" "*.Mask") (remove_unused_layers no)
   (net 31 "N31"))
  (pad "33" thru_hole circle (at 7.75 16.75) (size 1.524 1.524) (drill 0.762) (layers "*.Cu" "*.Mask") (remove_unused_layers no)
   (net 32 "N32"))
  (pad "34" thru_hole circle (at 10.25 16.75) (size 1.524 1.524) (drill 0.762) (layers "*.Cu" "*.Mask") (remove_unused_layers no)
   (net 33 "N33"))
  (pad "35" thru_hole circle (at 12.75 16.75) (size 1.524 1.524) (drill 0.762) (layers "*.Cu" "*.Mask") (remove_unused_layers no)
   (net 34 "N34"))
  (pad "36" thru_hole circle (at 15.25 16.75) (size 1.524 1.524) (drill 0.762) (layers "*.Cu" "*.Mask") (remove_unused_layers no)
   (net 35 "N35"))
  (pad "37" thru_hole circle (at 17.75 16.75) (size 1.524 1.524) (drill 0.762) (layers "*.Cu" "*.Mask") (remove_unused_layers no)
   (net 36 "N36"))
  (pad "38" thru_hole circle (at -14.738 16.75) (size 1.524 1.524) (drill 0.762) (layers "*.Cu" "*.Mask") (remove_unused_layers no)
   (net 1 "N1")))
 (gr_rect (start 129.5 43) (end 229 142.5) (locked yes) (stroke (width 0.05) (type default)) (fill none) (layer "Edge.Cuts"))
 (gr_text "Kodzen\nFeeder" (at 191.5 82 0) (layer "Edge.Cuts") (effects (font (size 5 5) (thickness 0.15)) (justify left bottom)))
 (segment (start 184.08 47.96) (end 183.62 47.5) (width 0.2) (layer "F.Cu") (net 14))
 (segment (start 222.5 47.96) (end 184.08 47.96) (width 0.2) (layer "F.Cu") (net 14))
 (segment (start 212.336 60.6645) (end 154.986 60.6645) (width 0.2) (layer "F.Cu") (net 15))
 (segment (start 222.5 50.5) (end 212.336 60.6645) (width 0.2) (layer "F.Cu") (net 15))
 (segment (start 154.986 60.6645) (end 152.5 63.15) (width 0.2) (layer "F.Cu") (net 15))
 (segment (start 151.608 108.132) (end 172.908 108.132) (width 0.2) (layer "F.Cu") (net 1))
 (segment (start 172.908 108.132) (end 173.758 107.282) (width 0.2) (layer "F.Cu") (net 1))
 (segment (start 138.222 93.19) (end 133 93.19) (width 0.2) (layer "F.Cu") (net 1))
 (segment (start 150.762 106.5) (end 150.762 107.286) (width 0.2) (layer "F.Cu") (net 1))
 (segment (start 173.758 106.5) (end 174.96 106.5) (width 0.2) (layer "F.Cu") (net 1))
 (segment (start 142.512 88.9) (end 138.222 93.19) (width 0.2) (layer "F.Cu") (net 1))
 (segment (start 150.762 107.286) (end 151.608 108.132) (width 0.2) (layer "F.Cu") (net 1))
 (segment (start 173.758 107.282) (end 173.758 106.5) (width 0.2) (layer "F.Cu") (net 1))
 (segment (start 149.56 106.5) (end 150.762 106.5) (width 0.2) (layer "F.Cu") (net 1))
 (segment (start 140.602 106.5) (end 140.602 107.326) (width 0.2) (layer "B.Cu") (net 1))
 (segment (start 139.4 106.5) (end 139.4 99.59) (width 0.2) (layer "B.Cu") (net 1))
 (segment (start 148.358 106.5) (end 149.56 106.5) (width 0.2) (layer "B.Cu") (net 1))
 (segment (start 139.4 106.5) (end 140.602 106.5) (width 0.2) (layer "B.Cu") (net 1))
 (segment (start 139.4 99.59) (end 133 93.19) (width 0.2) (layer "B.Cu") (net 1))
 (segment (start 148.358 107.286) (end 148.358 106.5) (width 0.2) (layer "B.Cu") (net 1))
 (segment (start 147.512 108.132) (end 148.358 107.286) (width 0.2) (layer "B.Cu") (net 1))
 (segment (start 140.602 107.326) (end 141.408 108.132) (width 0.2) (layer "B.Cu") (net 1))
 (segment (start 141.408 108.132) (end 147.512 108.132) (width 0.2) (layer "B.Cu") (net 1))
 (segment (start 167.34 103.74) (end 167.34 106.5) (width 0.2) (layer "B.Cu") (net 11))
 (segment (start 152.5 88.9) (end 167.34 103.74) (width 0.2) (layer "B.Cu") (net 11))
 (segment (start 138.79 100.81) (end 144.48 106.5) (width 0.2) (layer "F.Cu") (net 3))
 (segment (start 133 100.81) (end 138.79 100.81) (width 0.2) (layer "F.Cu") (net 3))
 (segment (start 143.142 106.5) (end 143.142 107.286) (width 0.2) (layer "F.Cu") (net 2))
 (segment (start 176.298 106.5) (end 177.5 106.5) (width 0.2) (layer "F.Cu") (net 2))
 (segment (start 144.39 108.534) (end 175.091 108.534) (width 0.2) (layer "F.Cu") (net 2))
 (segment (start 141.94 106.5) (end 143.142 106.5) (width 0.2) (layer "F.Cu") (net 2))
 (segment (start 143.142 107.286) (end 144.39 108.534) (width 0.2) (layer "F.Cu") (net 2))
 (segment (start 175.091 108.534) (end 176.298 107.326) (width 0.2) (layer "F.Cu") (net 2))
 (segment (start 176.298 107.326) (end 176.298 106.5) (width 0.2) (layer "F.Cu") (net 2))
 (segment (start 141.94 106.5) (end 141.94 90.84) (width 0.2) (layer "B.Cu") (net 2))
 (segment (start 141.94 90.84) (end 140 88.9) (width 0.2) (layer "B.Cu") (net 2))
 (segment (start 147.02 90.92) (end 145 88.9) (width 0.2) (layer "B.Cu") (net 4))
 (segment (start 147.02 106.5) (end 147.02 90.92) (width 0.2) (layer "B.Cu") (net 4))
 (segment (start 164.8 103.7) (end 164.8 106.5) (width 0.2) (layer "B.Cu") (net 10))
 (segment (start 150 88.9) (end 164.8 103.7) (width 0.2) (layer "B.Cu") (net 10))
 (segment (start 172.42 106.5) (end 172.42 103.82) (width 0.2) (layer "B.Cu") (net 13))
 (segment (start 172.42 103.82) (end 157.5 88.9) (width 0.2) (layer "B.Cu") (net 13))
 (segment (start 155 88.9) (end 169.88 103.78) (width 0.2) (layer "B.Cu") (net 12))
 (segment (start 169.88 103.78) (end 169.88 106.5) (width 0.2) (layer "B.Cu") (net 12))
 (segment (start 152.1 93.5) (end 152.1 106.5) (width 0.2) (layer "B.Cu") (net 5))
 (segment (start 147.5 88.9) (end 152.1 93.5) (width 0.2) (layer "B.Cu") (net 5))
 (segment (start 162.5 50) (end 162 49.5) (width 0.2) (layer "B.Cu") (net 18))
 (segment (start 168 50) (end 168.5 49.5) (width 0.2) (layer "B.Cu") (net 18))
 (segment (start 162.5 63.15) (end 162.5 50) (width 0.2) (layer "B.Cu") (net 18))
 (segment (start 162.5 50) (end 168 50) (width 0.2) (layer "B.Cu") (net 18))
 (segment (start 153.5 45) (end 162 45) (width 0.2) (layer "F.Cu") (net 17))
 (segment (start 149 49.5) (end 153.5 45) (width 0.2) (layer "F.Cu") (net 17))
 (segment (start 168.5 45) (end 162 45) (width 0.2) (layer "F.Cu") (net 17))
 (segment (start 171 47.5) (end 176 47.5) (width 0.2) (layer "F.Cu") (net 17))
 (segment (start 168.5 45) (end 171 47.5) (width 0.2) (layer "F.Cu") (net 17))
 (segment (start 148.988 49.512) (end 149 49.5) (width 0.2) (layer "B.Cu") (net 17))
 (segment (start 142.512 49.512) (end 148.988 49.512) (width 0.2) (layer "B.Cu") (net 17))
 (segment (start 142.512 63.15) (end 142.512 49.512) (width 0.2) (layer "B.Cu") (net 17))
 (segment (start 142.512 49.512) (end 142.5 49.5) (width 0.2) (layer "B.Cu") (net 17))
 (segment (start 149 45) (end 142.5 45) (width 0.2) (layer "F.Cu") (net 16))
 (segment (start 150.344 62.8062) (end 150.344 46.3438) (width 0.2) (layer "B.Cu") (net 16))
 (segment (start 150.344 46.3438) (end 149 45) (width 0.2) (layer "B.Cu") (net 16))
 (segment (start 150 63.15) (end 150.344 62.8062) (width 0.2) (layer "B.Cu") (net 16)))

